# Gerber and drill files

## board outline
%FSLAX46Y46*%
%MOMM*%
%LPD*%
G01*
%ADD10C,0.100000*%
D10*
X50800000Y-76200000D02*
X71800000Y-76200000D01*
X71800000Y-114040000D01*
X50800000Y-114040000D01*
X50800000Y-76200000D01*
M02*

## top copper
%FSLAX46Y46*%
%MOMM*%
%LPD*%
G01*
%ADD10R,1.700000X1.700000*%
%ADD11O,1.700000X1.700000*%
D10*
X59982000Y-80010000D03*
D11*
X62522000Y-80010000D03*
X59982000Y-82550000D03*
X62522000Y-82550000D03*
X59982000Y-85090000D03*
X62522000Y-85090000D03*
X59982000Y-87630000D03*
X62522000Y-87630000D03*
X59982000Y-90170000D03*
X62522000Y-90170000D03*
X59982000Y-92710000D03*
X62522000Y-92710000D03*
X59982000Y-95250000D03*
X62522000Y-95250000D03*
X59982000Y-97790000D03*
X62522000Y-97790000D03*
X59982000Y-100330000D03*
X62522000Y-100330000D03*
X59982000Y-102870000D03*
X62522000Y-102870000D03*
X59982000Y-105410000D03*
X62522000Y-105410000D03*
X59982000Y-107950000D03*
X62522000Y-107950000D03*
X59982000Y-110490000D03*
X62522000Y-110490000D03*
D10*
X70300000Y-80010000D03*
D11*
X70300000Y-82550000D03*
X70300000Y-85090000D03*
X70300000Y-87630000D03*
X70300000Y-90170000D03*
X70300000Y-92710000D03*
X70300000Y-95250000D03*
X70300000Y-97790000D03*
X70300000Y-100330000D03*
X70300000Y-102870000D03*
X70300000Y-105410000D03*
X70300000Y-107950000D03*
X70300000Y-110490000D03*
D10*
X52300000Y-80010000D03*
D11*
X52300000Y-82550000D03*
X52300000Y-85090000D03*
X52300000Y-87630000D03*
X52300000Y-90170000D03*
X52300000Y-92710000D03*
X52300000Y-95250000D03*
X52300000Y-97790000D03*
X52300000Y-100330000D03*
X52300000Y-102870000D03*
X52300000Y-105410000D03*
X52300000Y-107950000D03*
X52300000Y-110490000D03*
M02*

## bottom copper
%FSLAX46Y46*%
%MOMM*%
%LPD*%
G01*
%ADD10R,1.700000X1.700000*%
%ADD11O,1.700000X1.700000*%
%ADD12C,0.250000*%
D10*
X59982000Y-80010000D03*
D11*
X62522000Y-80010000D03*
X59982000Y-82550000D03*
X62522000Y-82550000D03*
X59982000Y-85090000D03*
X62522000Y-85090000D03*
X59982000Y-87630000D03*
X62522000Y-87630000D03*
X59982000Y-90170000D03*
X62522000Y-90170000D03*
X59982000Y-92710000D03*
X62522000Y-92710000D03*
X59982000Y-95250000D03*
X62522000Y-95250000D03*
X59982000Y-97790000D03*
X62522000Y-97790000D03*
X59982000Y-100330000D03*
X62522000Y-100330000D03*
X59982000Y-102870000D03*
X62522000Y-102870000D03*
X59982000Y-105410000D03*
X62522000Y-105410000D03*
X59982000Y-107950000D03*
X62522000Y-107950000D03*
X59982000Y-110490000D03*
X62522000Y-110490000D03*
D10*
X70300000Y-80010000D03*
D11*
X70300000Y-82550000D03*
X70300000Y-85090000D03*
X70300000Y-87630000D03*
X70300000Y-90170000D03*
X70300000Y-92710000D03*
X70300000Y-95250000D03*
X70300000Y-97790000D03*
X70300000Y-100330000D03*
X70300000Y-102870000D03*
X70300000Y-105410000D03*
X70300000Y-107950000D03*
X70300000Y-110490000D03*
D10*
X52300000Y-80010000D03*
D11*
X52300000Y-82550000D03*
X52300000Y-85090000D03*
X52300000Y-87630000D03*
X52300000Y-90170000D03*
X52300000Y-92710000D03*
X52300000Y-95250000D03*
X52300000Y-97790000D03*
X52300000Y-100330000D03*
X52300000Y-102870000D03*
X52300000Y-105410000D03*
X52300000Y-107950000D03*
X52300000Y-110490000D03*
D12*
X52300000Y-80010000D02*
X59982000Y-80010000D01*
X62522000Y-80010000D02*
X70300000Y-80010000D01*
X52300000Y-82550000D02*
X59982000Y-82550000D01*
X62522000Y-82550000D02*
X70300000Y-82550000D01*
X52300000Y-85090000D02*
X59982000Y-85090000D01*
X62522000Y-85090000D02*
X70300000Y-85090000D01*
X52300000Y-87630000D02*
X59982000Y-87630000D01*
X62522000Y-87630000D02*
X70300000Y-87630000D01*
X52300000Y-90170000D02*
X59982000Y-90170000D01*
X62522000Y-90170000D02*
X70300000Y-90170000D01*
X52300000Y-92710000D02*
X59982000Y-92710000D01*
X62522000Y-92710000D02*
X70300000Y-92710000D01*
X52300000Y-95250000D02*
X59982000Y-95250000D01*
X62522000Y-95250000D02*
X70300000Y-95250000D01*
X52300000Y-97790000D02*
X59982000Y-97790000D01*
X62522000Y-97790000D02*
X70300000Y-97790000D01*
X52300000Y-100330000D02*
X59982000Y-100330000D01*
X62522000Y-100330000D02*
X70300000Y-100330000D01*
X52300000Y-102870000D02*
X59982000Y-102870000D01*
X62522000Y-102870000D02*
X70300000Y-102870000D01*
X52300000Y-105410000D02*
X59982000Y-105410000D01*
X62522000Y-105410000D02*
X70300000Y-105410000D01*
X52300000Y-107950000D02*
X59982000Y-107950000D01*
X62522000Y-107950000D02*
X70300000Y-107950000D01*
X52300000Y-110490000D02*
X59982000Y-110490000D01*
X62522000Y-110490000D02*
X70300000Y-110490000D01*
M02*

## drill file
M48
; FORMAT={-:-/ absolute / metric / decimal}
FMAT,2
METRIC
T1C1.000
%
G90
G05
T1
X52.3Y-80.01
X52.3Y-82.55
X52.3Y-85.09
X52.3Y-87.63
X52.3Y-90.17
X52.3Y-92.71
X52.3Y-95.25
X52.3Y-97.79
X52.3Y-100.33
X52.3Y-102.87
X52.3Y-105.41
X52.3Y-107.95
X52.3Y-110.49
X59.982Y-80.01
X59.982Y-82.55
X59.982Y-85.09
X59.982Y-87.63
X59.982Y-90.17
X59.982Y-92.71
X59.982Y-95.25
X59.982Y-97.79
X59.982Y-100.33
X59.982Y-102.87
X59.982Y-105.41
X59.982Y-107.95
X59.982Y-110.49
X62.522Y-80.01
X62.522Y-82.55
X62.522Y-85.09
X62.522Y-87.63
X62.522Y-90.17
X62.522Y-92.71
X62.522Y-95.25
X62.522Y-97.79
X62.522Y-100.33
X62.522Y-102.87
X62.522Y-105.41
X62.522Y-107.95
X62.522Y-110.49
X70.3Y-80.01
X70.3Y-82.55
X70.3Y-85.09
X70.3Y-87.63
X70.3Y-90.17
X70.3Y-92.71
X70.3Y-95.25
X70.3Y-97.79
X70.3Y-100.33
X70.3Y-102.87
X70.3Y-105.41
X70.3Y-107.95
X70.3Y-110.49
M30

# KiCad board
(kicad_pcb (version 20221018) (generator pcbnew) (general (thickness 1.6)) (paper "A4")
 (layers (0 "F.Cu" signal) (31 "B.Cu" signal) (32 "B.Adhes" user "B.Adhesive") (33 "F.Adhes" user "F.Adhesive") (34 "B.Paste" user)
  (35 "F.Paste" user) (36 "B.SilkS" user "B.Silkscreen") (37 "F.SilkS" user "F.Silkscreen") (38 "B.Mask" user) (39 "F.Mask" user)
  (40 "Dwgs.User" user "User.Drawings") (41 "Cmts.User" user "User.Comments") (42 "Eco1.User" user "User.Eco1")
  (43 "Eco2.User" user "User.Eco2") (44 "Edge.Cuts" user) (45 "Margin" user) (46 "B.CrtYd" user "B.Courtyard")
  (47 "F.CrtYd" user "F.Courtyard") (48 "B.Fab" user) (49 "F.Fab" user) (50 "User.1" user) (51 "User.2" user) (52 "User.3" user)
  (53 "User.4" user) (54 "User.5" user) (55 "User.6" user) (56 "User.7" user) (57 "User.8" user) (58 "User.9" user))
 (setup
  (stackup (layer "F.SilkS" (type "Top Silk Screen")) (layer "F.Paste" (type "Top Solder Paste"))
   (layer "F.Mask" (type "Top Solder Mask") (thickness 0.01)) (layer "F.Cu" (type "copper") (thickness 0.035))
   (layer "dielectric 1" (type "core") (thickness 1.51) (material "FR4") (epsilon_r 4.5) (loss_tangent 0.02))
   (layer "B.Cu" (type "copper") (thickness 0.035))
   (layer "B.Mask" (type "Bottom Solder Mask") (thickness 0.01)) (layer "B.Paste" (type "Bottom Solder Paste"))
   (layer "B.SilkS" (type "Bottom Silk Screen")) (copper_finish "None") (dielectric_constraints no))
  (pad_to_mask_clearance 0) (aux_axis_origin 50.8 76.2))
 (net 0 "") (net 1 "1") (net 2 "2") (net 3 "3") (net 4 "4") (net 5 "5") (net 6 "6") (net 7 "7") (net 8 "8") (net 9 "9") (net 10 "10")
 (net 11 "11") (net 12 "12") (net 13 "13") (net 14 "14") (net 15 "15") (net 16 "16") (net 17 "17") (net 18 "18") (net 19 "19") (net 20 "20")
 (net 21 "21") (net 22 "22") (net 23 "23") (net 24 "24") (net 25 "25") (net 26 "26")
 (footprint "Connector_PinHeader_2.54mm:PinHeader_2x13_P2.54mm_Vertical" (layer "F.Cu") (at 59.982 80.01)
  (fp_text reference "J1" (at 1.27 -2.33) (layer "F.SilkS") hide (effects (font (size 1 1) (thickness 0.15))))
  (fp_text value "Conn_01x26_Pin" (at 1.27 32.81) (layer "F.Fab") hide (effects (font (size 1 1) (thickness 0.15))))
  (pad "1" thru_hole rect (at 0 0) (size 1.7 1.7) (drill 1) (layers "*.Cu" "*.Mask") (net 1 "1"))
  (pad "2" thru_hole oval (at 2.54 0) (size 1.7 1.7) (drill 1) (layers "*.Cu" "*.Mask") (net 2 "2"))
  (pad "3" thru_hole oval (at 0 2.54) (size 1.7 1.7) (drill 1) (layers "*.Cu" "*.Mask") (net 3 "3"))
  (pad "4" thru_hole oval (at 2.54 2.54) (size 1.7 1.7) (drill 1) (layers "*.Cu" "*.Mask") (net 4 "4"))
  (pad "5" thru_hole oval (at 0 5.08) (size 1.7 1.7) (drill 1) (layers "*.Cu" "*.Mask") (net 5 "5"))
  (pad "6" thru_hole oval (at 2.54 5.08) (size 1.7 1.7) (drill 1) (layers "*.Cu" "*.Mask") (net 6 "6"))
  (pad "7" thru_hole oval (at 0 7.62) (size 1.7 1.7) (drill 1) (layers "*.Cu" "*.Mask") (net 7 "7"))
  (pad "8" thru_hole oval (at 2.54 7.62) (size 1.7 1.7) (drill 1) (layers "*.Cu" "*.Mask") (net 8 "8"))
  (pad "9" thru_hole oval (at 0 10.16) (size 1.7 1.7) (drill 1) (layers "*.Cu" "*.Mask") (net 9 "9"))
  (pad "10" thru_hole oval (at 2.54 10.16) (size 1.7 1.7) (drill 1) (layers "*.Cu" "*.Mask") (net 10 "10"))
  (pad "11" thru_hole oval (at 0 12.7) (size 1.7 1.7) (drill 1) (layers "*.Cu" "*.Mask") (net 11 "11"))
  (pad "12" thru_hole oval (at 2.54 12.7) (size 1.7 1.7) (drill 1) (layers "*.Cu" "*.Mask") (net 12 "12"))
  (pad "13" thru_hole oval (at 0 15.24) (size 1.7 1.7) (drill 1) (layers "*.Cu" "*.Mask") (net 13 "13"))
  (pad "14" thru_hole oval (at 2.54 15.24) (size 1.7 1.7) (drill 1) (layers "*.Cu" "*.Mask") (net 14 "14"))
  (pad "15" thru_hole oval (at 0 17.78) (size 1.7 1.7) (drill 1) (layers "*.Cu" "*.Mask") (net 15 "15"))
  (pad "16" thru_hole oval (at 2.54 17.78) (size 1.7 1.7) (drill 1) (layers "*.Cu" "*.Mask") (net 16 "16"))
  (pad "17" thru_hole oval (at 0 20.32) (size 1.7 1.7) (drill 1) (layers "*.Cu" "*.Mask") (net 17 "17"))
  (pad "18" thru_hole oval (at 2.54 20.32) (size 1.7 1.7) (drill 1) (layers "*.Cu" "*.Mask") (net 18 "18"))
  (pad "19" thru_hole oval (at 0 22.86) (size 1.7 1.7) (drill 1) (layers "*.Cu" "*.Mask") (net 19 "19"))
  (pad "20" thru_hole oval (at 2.54 22.86) (size 1.7 1.7) (drill 1) (layers "*.Cu" "*.Mask") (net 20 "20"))
  (pad "21" thru_hole oval (at 0 25.4) (size 1.7 1.7) (drill 1) (layers "*.Cu" "*.Mask") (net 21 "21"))
  (pad "22" thru_hole oval (at 2.54 25.4) (size 1.7 1.7) (drill 1) (layers "*.Cu" "*.Mask") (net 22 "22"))
  (pad "23" thru_hole oval (at 0 27.94) (size 1.7 1.7) (drill 1) (layers "*.Cu" "*.Mask") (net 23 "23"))
  (pad "24" thru_hole oval (at 2.54 27.94) (size 1.7 1.7) (drill 1) (layers "*.Cu" "*.Mask") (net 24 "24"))
  (pad "25" thru_hole oval (at 0 30.48) (size 1.7 1.7) (drill 1) (layers "*.Cu" "*.Mask") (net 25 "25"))
  (pad "26" thru_hole oval (at 2.54 30.48) (size 1.7 1.7) (drill 1) (layers "*.Cu" "*.Mask") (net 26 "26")))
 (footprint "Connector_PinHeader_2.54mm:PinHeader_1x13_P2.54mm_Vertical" (layer "B.Cu") (at 70.3 80.01 180)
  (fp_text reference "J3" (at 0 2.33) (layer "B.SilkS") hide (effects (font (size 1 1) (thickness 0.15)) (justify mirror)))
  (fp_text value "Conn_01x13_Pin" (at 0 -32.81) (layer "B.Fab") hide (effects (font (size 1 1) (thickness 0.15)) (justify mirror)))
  (pad "1" thru_hole rect (at 0 0 180) (size 1.7 1.7) (drill 1) (layers "*.Cu" "*.Mask") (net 2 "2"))
  (pad "2" thru_hole oval (at 0 -2.54 180) (size 1.7 1.7) (drill 1) (layers "*.Cu" "*.Mask") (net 4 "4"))
  (pad "3" thru_hole oval (at 0 -5.08 180) (size 1.7 1.7) (drill 1) (layers "*.Cu" "*.Mask") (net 6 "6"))
  (pad "4" thru_hole oval (at 0 -7.62 180) (size 1.7 1.7) (drill 1) (layers "*.Cu" "*.Mask") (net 8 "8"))
  (pad "5" thru_hole oval (at 0 -10.16 180) (size 1.7 1.7) (drill 1) (layers "*.Cu" "*.Mask") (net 10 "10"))
  (pad "6" thru_hole oval (at 0 -12.7 180) (size 1.7 1.7) (drill 1) (layers "*.Cu" "*.Mask") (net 12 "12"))
  (pad "7" thru_hole oval (at 0 -15.24 180) (size 1.7 1.7) (drill 1) (layers "*.Cu" "*.Mask") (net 14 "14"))
  (pad "8" thru_hole oval (at 0 -17.78 180) (size 1.7 1.7) (drill 1) (layers "*.Cu" "*.Mask") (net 16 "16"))
  (pad "9" thru_hole oval (at 0 -20.32 180) (size 1.7 1.7) (drill 1) (layers "*.Cu" "*.Mask") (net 18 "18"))
  (pad "10" thru_hole oval (at 0 -22.86 180) (size 1.7 1.7) (drill 1) (layers "*.Cu" "*.Mask") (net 20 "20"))
  (pad "11" thru_hole oval (at 0 -25.4 180) (size 1.7 1.7) (drill 1) (layers "*.Cu" "*.Mask") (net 22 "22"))
  (pad "12" thru_hole oval (at 0 -27.94 180) (size 1.7 1.7) (drill 1) (layers "*.Cu" "*.Mask") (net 24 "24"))
  (pad "13" thru_hole oval (at 0 -30.48 180) (size 1.7 1.7) (drill 1) (layers "*.Cu" "*.Mask") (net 26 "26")))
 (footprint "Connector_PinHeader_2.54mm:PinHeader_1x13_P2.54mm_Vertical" (layer "B.Cu") (at 52.3 80.01 180)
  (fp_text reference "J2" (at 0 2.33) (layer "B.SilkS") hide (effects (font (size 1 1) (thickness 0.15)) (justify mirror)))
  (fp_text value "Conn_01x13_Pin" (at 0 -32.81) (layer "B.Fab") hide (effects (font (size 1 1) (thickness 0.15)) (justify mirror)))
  (pad "1" thru_hole rect (at 0 0 180) (size 1.7 1.7) (drill 1) (layers "*.Cu" "*.Mask") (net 1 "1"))
  (pad "2" thru_hole oval (at 0 -2.54 180) (size 1.7 1.7) (drill 1) (layers "*.Cu" "*.Mask") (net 3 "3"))
  (pad "3" thru_hole oval (at 0 -5.08 180) (size 1.7 1.7) (drill 1) (layers "*.Cu" "*.Mask") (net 5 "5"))
  (pad "4" thru_hole oval (at 0 -7.62 180) (size 1.7 1.7) (drill 1) (layers "*.Cu" "*.Mask") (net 7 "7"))
  (pad "5" thru_hole oval (at 0 -10.16 180) (size 1.7 1.7) (drill 1) (layers "*.Cu" "*.Mask") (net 9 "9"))
  (pad "6" thru_hole oval (at 0 -12.7 180) (size 1.7 1.7) (drill 1) (layers "*.Cu" "*.Mask") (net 11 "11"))
  (pad "7" thru_hole oval (at 0 -15.24 180) (size 1.7 1.7) (drill 1) (layers "*.Cu" "*.Mask") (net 13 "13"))
  (pad "8" thru_hole oval (at 0 -17.78 180) (size 1.7 1.7) (drill 1) (layers "*.Cu" "*.Mask") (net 15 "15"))
  (pad "9" thru_hole oval (at 0 -20.32 180) (size 1.7 1.7) (drill 1) (layers "*.Cu" "*.Mask") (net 17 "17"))
  (pad "10" thru_hole oval (at 0 -22.86 180) (size 1.7 1.7) (drill 1) (layers "*.Cu" "*.Mask") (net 19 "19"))
  (pad "11" thru_hole oval (at 0 -25.4 180) (size 1.7 1.7) (drill 1) (layers "*.Cu" "*.Mask") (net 21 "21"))
  (pad "12" thru_hole oval (at 0 -27.94 180) (size 1.7 1.7) (drill 1) (layers "*.Cu" "*.Mask") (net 23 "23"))
  (pad "13" thru_hole oval (at 0 -30.48 180) (size 1.7 1.7) (drill 1) (layers "*.Cu" "*.Mask") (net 25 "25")))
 (gr_rect (start 50.8 76.2) (end 71.8 114.04) (stroke (width 0.1) (type default)) (fill none) (layer "Edge.Cuts"))
 (segment (start 52.3 80.01) (end 59.982 80.01) (width 0.25) (layer "B.Cu") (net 1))
 (segment (start 62.522 80.01) (end 70.3 80.01) (width 0.25) (layer "B.Cu") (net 2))
 (segment (start 52.3 82.55) (end 59.982 82.55) (width 0.25) (layer "B.Cu") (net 3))
 (segment (start 62.522 82.55) (end 70.3 82.55) (width 0.25) (layer "B.Cu") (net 4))
 (segment (start 52.3 85.09) (end 59.982 85.09) (width 0.25) (layer "B.Cu") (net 5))
 (segment (start 62.522 85.09) (end 70.3 85.09) (width 0.25) (layer "B.Cu") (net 6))
 (segment (start 52.3 87.63) (end 59.982 87.63) (width 0.25) (layer "B.Cu") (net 7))
 (segment (start 62.522 87.63) (end 70.3 87.63) (width 0.25) (layer "B.Cu") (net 8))
 (segment (start 52.3 90.17) (end 59.982 90.17) (width 0.25) (layer "B.Cu") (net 9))
 (segment (start 62.522 90.17) (end 70.3 90.17) (width 0.25) (layer "B.Cu") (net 10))
 (segment (start 52.3 92.71) (end 59.982 92.71) (width 0.25) (layer "B.Cu") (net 11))
 (segment (start 62.522 92.71) (end 70.3 92.71) (width 0.25) (layer "B.Cu") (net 12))
 (segment (start 52.3 95.25) (end 59.982 95.25) (width 0.25) (layer "B.Cu") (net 13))
 (segment (start 62.522 95.25) (end 70.3 95.25) (width 0.25) (layer "B.Cu") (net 14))
 (segment (start 52.3 97.79) (end 59.982 97.79) (width 0.25) (layer "B.Cu") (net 15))
 (segment (start 62.522 97.79) (end 70.3 97.79) (width 0.25) (layer "B.Cu") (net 16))
 (segment (start 52.3 100.33) (end 59.982 100.33) (width 0.25) (layer "B.Cu") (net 17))
 (segment (start 62.522 100.33) (end 70.3 100.33) (width 0.25) (layer "B.Cu") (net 18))
 (segment (start 52.3 102.87) (end 59.982 102.87) (width 0.25) (layer "B.Cu") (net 19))
 (segment (start 62.522 102.87) (end 70.3 102.87) (width 0.25) (layer "B.Cu") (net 20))
 (segment (start 52.3 105.41) (end 59.982 105.41) (width 0.25) (layer "B.Cu") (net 21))
 (segment (start 62.522 105.41) (end 70.3 105.41) (width 0.25) (layer "B.Cu") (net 22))
 (segment (start 52.3 107.95) (end 59.982 107.95) (width 0.25) (layer "B.Cu") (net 23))
 (segment (start 62.522 107.95) (end 70.3 107.95) (width 0.25) (layer "B.Cu") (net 24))
 (segment (start 52.3 110.49) (end 59.982 110.49) (width 0.25) (layer "B.Cu") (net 25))
 (segment (start 62.522 110.49) (end 70.3 110.49) (width 0.25) (layer "B.Cu") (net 26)))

